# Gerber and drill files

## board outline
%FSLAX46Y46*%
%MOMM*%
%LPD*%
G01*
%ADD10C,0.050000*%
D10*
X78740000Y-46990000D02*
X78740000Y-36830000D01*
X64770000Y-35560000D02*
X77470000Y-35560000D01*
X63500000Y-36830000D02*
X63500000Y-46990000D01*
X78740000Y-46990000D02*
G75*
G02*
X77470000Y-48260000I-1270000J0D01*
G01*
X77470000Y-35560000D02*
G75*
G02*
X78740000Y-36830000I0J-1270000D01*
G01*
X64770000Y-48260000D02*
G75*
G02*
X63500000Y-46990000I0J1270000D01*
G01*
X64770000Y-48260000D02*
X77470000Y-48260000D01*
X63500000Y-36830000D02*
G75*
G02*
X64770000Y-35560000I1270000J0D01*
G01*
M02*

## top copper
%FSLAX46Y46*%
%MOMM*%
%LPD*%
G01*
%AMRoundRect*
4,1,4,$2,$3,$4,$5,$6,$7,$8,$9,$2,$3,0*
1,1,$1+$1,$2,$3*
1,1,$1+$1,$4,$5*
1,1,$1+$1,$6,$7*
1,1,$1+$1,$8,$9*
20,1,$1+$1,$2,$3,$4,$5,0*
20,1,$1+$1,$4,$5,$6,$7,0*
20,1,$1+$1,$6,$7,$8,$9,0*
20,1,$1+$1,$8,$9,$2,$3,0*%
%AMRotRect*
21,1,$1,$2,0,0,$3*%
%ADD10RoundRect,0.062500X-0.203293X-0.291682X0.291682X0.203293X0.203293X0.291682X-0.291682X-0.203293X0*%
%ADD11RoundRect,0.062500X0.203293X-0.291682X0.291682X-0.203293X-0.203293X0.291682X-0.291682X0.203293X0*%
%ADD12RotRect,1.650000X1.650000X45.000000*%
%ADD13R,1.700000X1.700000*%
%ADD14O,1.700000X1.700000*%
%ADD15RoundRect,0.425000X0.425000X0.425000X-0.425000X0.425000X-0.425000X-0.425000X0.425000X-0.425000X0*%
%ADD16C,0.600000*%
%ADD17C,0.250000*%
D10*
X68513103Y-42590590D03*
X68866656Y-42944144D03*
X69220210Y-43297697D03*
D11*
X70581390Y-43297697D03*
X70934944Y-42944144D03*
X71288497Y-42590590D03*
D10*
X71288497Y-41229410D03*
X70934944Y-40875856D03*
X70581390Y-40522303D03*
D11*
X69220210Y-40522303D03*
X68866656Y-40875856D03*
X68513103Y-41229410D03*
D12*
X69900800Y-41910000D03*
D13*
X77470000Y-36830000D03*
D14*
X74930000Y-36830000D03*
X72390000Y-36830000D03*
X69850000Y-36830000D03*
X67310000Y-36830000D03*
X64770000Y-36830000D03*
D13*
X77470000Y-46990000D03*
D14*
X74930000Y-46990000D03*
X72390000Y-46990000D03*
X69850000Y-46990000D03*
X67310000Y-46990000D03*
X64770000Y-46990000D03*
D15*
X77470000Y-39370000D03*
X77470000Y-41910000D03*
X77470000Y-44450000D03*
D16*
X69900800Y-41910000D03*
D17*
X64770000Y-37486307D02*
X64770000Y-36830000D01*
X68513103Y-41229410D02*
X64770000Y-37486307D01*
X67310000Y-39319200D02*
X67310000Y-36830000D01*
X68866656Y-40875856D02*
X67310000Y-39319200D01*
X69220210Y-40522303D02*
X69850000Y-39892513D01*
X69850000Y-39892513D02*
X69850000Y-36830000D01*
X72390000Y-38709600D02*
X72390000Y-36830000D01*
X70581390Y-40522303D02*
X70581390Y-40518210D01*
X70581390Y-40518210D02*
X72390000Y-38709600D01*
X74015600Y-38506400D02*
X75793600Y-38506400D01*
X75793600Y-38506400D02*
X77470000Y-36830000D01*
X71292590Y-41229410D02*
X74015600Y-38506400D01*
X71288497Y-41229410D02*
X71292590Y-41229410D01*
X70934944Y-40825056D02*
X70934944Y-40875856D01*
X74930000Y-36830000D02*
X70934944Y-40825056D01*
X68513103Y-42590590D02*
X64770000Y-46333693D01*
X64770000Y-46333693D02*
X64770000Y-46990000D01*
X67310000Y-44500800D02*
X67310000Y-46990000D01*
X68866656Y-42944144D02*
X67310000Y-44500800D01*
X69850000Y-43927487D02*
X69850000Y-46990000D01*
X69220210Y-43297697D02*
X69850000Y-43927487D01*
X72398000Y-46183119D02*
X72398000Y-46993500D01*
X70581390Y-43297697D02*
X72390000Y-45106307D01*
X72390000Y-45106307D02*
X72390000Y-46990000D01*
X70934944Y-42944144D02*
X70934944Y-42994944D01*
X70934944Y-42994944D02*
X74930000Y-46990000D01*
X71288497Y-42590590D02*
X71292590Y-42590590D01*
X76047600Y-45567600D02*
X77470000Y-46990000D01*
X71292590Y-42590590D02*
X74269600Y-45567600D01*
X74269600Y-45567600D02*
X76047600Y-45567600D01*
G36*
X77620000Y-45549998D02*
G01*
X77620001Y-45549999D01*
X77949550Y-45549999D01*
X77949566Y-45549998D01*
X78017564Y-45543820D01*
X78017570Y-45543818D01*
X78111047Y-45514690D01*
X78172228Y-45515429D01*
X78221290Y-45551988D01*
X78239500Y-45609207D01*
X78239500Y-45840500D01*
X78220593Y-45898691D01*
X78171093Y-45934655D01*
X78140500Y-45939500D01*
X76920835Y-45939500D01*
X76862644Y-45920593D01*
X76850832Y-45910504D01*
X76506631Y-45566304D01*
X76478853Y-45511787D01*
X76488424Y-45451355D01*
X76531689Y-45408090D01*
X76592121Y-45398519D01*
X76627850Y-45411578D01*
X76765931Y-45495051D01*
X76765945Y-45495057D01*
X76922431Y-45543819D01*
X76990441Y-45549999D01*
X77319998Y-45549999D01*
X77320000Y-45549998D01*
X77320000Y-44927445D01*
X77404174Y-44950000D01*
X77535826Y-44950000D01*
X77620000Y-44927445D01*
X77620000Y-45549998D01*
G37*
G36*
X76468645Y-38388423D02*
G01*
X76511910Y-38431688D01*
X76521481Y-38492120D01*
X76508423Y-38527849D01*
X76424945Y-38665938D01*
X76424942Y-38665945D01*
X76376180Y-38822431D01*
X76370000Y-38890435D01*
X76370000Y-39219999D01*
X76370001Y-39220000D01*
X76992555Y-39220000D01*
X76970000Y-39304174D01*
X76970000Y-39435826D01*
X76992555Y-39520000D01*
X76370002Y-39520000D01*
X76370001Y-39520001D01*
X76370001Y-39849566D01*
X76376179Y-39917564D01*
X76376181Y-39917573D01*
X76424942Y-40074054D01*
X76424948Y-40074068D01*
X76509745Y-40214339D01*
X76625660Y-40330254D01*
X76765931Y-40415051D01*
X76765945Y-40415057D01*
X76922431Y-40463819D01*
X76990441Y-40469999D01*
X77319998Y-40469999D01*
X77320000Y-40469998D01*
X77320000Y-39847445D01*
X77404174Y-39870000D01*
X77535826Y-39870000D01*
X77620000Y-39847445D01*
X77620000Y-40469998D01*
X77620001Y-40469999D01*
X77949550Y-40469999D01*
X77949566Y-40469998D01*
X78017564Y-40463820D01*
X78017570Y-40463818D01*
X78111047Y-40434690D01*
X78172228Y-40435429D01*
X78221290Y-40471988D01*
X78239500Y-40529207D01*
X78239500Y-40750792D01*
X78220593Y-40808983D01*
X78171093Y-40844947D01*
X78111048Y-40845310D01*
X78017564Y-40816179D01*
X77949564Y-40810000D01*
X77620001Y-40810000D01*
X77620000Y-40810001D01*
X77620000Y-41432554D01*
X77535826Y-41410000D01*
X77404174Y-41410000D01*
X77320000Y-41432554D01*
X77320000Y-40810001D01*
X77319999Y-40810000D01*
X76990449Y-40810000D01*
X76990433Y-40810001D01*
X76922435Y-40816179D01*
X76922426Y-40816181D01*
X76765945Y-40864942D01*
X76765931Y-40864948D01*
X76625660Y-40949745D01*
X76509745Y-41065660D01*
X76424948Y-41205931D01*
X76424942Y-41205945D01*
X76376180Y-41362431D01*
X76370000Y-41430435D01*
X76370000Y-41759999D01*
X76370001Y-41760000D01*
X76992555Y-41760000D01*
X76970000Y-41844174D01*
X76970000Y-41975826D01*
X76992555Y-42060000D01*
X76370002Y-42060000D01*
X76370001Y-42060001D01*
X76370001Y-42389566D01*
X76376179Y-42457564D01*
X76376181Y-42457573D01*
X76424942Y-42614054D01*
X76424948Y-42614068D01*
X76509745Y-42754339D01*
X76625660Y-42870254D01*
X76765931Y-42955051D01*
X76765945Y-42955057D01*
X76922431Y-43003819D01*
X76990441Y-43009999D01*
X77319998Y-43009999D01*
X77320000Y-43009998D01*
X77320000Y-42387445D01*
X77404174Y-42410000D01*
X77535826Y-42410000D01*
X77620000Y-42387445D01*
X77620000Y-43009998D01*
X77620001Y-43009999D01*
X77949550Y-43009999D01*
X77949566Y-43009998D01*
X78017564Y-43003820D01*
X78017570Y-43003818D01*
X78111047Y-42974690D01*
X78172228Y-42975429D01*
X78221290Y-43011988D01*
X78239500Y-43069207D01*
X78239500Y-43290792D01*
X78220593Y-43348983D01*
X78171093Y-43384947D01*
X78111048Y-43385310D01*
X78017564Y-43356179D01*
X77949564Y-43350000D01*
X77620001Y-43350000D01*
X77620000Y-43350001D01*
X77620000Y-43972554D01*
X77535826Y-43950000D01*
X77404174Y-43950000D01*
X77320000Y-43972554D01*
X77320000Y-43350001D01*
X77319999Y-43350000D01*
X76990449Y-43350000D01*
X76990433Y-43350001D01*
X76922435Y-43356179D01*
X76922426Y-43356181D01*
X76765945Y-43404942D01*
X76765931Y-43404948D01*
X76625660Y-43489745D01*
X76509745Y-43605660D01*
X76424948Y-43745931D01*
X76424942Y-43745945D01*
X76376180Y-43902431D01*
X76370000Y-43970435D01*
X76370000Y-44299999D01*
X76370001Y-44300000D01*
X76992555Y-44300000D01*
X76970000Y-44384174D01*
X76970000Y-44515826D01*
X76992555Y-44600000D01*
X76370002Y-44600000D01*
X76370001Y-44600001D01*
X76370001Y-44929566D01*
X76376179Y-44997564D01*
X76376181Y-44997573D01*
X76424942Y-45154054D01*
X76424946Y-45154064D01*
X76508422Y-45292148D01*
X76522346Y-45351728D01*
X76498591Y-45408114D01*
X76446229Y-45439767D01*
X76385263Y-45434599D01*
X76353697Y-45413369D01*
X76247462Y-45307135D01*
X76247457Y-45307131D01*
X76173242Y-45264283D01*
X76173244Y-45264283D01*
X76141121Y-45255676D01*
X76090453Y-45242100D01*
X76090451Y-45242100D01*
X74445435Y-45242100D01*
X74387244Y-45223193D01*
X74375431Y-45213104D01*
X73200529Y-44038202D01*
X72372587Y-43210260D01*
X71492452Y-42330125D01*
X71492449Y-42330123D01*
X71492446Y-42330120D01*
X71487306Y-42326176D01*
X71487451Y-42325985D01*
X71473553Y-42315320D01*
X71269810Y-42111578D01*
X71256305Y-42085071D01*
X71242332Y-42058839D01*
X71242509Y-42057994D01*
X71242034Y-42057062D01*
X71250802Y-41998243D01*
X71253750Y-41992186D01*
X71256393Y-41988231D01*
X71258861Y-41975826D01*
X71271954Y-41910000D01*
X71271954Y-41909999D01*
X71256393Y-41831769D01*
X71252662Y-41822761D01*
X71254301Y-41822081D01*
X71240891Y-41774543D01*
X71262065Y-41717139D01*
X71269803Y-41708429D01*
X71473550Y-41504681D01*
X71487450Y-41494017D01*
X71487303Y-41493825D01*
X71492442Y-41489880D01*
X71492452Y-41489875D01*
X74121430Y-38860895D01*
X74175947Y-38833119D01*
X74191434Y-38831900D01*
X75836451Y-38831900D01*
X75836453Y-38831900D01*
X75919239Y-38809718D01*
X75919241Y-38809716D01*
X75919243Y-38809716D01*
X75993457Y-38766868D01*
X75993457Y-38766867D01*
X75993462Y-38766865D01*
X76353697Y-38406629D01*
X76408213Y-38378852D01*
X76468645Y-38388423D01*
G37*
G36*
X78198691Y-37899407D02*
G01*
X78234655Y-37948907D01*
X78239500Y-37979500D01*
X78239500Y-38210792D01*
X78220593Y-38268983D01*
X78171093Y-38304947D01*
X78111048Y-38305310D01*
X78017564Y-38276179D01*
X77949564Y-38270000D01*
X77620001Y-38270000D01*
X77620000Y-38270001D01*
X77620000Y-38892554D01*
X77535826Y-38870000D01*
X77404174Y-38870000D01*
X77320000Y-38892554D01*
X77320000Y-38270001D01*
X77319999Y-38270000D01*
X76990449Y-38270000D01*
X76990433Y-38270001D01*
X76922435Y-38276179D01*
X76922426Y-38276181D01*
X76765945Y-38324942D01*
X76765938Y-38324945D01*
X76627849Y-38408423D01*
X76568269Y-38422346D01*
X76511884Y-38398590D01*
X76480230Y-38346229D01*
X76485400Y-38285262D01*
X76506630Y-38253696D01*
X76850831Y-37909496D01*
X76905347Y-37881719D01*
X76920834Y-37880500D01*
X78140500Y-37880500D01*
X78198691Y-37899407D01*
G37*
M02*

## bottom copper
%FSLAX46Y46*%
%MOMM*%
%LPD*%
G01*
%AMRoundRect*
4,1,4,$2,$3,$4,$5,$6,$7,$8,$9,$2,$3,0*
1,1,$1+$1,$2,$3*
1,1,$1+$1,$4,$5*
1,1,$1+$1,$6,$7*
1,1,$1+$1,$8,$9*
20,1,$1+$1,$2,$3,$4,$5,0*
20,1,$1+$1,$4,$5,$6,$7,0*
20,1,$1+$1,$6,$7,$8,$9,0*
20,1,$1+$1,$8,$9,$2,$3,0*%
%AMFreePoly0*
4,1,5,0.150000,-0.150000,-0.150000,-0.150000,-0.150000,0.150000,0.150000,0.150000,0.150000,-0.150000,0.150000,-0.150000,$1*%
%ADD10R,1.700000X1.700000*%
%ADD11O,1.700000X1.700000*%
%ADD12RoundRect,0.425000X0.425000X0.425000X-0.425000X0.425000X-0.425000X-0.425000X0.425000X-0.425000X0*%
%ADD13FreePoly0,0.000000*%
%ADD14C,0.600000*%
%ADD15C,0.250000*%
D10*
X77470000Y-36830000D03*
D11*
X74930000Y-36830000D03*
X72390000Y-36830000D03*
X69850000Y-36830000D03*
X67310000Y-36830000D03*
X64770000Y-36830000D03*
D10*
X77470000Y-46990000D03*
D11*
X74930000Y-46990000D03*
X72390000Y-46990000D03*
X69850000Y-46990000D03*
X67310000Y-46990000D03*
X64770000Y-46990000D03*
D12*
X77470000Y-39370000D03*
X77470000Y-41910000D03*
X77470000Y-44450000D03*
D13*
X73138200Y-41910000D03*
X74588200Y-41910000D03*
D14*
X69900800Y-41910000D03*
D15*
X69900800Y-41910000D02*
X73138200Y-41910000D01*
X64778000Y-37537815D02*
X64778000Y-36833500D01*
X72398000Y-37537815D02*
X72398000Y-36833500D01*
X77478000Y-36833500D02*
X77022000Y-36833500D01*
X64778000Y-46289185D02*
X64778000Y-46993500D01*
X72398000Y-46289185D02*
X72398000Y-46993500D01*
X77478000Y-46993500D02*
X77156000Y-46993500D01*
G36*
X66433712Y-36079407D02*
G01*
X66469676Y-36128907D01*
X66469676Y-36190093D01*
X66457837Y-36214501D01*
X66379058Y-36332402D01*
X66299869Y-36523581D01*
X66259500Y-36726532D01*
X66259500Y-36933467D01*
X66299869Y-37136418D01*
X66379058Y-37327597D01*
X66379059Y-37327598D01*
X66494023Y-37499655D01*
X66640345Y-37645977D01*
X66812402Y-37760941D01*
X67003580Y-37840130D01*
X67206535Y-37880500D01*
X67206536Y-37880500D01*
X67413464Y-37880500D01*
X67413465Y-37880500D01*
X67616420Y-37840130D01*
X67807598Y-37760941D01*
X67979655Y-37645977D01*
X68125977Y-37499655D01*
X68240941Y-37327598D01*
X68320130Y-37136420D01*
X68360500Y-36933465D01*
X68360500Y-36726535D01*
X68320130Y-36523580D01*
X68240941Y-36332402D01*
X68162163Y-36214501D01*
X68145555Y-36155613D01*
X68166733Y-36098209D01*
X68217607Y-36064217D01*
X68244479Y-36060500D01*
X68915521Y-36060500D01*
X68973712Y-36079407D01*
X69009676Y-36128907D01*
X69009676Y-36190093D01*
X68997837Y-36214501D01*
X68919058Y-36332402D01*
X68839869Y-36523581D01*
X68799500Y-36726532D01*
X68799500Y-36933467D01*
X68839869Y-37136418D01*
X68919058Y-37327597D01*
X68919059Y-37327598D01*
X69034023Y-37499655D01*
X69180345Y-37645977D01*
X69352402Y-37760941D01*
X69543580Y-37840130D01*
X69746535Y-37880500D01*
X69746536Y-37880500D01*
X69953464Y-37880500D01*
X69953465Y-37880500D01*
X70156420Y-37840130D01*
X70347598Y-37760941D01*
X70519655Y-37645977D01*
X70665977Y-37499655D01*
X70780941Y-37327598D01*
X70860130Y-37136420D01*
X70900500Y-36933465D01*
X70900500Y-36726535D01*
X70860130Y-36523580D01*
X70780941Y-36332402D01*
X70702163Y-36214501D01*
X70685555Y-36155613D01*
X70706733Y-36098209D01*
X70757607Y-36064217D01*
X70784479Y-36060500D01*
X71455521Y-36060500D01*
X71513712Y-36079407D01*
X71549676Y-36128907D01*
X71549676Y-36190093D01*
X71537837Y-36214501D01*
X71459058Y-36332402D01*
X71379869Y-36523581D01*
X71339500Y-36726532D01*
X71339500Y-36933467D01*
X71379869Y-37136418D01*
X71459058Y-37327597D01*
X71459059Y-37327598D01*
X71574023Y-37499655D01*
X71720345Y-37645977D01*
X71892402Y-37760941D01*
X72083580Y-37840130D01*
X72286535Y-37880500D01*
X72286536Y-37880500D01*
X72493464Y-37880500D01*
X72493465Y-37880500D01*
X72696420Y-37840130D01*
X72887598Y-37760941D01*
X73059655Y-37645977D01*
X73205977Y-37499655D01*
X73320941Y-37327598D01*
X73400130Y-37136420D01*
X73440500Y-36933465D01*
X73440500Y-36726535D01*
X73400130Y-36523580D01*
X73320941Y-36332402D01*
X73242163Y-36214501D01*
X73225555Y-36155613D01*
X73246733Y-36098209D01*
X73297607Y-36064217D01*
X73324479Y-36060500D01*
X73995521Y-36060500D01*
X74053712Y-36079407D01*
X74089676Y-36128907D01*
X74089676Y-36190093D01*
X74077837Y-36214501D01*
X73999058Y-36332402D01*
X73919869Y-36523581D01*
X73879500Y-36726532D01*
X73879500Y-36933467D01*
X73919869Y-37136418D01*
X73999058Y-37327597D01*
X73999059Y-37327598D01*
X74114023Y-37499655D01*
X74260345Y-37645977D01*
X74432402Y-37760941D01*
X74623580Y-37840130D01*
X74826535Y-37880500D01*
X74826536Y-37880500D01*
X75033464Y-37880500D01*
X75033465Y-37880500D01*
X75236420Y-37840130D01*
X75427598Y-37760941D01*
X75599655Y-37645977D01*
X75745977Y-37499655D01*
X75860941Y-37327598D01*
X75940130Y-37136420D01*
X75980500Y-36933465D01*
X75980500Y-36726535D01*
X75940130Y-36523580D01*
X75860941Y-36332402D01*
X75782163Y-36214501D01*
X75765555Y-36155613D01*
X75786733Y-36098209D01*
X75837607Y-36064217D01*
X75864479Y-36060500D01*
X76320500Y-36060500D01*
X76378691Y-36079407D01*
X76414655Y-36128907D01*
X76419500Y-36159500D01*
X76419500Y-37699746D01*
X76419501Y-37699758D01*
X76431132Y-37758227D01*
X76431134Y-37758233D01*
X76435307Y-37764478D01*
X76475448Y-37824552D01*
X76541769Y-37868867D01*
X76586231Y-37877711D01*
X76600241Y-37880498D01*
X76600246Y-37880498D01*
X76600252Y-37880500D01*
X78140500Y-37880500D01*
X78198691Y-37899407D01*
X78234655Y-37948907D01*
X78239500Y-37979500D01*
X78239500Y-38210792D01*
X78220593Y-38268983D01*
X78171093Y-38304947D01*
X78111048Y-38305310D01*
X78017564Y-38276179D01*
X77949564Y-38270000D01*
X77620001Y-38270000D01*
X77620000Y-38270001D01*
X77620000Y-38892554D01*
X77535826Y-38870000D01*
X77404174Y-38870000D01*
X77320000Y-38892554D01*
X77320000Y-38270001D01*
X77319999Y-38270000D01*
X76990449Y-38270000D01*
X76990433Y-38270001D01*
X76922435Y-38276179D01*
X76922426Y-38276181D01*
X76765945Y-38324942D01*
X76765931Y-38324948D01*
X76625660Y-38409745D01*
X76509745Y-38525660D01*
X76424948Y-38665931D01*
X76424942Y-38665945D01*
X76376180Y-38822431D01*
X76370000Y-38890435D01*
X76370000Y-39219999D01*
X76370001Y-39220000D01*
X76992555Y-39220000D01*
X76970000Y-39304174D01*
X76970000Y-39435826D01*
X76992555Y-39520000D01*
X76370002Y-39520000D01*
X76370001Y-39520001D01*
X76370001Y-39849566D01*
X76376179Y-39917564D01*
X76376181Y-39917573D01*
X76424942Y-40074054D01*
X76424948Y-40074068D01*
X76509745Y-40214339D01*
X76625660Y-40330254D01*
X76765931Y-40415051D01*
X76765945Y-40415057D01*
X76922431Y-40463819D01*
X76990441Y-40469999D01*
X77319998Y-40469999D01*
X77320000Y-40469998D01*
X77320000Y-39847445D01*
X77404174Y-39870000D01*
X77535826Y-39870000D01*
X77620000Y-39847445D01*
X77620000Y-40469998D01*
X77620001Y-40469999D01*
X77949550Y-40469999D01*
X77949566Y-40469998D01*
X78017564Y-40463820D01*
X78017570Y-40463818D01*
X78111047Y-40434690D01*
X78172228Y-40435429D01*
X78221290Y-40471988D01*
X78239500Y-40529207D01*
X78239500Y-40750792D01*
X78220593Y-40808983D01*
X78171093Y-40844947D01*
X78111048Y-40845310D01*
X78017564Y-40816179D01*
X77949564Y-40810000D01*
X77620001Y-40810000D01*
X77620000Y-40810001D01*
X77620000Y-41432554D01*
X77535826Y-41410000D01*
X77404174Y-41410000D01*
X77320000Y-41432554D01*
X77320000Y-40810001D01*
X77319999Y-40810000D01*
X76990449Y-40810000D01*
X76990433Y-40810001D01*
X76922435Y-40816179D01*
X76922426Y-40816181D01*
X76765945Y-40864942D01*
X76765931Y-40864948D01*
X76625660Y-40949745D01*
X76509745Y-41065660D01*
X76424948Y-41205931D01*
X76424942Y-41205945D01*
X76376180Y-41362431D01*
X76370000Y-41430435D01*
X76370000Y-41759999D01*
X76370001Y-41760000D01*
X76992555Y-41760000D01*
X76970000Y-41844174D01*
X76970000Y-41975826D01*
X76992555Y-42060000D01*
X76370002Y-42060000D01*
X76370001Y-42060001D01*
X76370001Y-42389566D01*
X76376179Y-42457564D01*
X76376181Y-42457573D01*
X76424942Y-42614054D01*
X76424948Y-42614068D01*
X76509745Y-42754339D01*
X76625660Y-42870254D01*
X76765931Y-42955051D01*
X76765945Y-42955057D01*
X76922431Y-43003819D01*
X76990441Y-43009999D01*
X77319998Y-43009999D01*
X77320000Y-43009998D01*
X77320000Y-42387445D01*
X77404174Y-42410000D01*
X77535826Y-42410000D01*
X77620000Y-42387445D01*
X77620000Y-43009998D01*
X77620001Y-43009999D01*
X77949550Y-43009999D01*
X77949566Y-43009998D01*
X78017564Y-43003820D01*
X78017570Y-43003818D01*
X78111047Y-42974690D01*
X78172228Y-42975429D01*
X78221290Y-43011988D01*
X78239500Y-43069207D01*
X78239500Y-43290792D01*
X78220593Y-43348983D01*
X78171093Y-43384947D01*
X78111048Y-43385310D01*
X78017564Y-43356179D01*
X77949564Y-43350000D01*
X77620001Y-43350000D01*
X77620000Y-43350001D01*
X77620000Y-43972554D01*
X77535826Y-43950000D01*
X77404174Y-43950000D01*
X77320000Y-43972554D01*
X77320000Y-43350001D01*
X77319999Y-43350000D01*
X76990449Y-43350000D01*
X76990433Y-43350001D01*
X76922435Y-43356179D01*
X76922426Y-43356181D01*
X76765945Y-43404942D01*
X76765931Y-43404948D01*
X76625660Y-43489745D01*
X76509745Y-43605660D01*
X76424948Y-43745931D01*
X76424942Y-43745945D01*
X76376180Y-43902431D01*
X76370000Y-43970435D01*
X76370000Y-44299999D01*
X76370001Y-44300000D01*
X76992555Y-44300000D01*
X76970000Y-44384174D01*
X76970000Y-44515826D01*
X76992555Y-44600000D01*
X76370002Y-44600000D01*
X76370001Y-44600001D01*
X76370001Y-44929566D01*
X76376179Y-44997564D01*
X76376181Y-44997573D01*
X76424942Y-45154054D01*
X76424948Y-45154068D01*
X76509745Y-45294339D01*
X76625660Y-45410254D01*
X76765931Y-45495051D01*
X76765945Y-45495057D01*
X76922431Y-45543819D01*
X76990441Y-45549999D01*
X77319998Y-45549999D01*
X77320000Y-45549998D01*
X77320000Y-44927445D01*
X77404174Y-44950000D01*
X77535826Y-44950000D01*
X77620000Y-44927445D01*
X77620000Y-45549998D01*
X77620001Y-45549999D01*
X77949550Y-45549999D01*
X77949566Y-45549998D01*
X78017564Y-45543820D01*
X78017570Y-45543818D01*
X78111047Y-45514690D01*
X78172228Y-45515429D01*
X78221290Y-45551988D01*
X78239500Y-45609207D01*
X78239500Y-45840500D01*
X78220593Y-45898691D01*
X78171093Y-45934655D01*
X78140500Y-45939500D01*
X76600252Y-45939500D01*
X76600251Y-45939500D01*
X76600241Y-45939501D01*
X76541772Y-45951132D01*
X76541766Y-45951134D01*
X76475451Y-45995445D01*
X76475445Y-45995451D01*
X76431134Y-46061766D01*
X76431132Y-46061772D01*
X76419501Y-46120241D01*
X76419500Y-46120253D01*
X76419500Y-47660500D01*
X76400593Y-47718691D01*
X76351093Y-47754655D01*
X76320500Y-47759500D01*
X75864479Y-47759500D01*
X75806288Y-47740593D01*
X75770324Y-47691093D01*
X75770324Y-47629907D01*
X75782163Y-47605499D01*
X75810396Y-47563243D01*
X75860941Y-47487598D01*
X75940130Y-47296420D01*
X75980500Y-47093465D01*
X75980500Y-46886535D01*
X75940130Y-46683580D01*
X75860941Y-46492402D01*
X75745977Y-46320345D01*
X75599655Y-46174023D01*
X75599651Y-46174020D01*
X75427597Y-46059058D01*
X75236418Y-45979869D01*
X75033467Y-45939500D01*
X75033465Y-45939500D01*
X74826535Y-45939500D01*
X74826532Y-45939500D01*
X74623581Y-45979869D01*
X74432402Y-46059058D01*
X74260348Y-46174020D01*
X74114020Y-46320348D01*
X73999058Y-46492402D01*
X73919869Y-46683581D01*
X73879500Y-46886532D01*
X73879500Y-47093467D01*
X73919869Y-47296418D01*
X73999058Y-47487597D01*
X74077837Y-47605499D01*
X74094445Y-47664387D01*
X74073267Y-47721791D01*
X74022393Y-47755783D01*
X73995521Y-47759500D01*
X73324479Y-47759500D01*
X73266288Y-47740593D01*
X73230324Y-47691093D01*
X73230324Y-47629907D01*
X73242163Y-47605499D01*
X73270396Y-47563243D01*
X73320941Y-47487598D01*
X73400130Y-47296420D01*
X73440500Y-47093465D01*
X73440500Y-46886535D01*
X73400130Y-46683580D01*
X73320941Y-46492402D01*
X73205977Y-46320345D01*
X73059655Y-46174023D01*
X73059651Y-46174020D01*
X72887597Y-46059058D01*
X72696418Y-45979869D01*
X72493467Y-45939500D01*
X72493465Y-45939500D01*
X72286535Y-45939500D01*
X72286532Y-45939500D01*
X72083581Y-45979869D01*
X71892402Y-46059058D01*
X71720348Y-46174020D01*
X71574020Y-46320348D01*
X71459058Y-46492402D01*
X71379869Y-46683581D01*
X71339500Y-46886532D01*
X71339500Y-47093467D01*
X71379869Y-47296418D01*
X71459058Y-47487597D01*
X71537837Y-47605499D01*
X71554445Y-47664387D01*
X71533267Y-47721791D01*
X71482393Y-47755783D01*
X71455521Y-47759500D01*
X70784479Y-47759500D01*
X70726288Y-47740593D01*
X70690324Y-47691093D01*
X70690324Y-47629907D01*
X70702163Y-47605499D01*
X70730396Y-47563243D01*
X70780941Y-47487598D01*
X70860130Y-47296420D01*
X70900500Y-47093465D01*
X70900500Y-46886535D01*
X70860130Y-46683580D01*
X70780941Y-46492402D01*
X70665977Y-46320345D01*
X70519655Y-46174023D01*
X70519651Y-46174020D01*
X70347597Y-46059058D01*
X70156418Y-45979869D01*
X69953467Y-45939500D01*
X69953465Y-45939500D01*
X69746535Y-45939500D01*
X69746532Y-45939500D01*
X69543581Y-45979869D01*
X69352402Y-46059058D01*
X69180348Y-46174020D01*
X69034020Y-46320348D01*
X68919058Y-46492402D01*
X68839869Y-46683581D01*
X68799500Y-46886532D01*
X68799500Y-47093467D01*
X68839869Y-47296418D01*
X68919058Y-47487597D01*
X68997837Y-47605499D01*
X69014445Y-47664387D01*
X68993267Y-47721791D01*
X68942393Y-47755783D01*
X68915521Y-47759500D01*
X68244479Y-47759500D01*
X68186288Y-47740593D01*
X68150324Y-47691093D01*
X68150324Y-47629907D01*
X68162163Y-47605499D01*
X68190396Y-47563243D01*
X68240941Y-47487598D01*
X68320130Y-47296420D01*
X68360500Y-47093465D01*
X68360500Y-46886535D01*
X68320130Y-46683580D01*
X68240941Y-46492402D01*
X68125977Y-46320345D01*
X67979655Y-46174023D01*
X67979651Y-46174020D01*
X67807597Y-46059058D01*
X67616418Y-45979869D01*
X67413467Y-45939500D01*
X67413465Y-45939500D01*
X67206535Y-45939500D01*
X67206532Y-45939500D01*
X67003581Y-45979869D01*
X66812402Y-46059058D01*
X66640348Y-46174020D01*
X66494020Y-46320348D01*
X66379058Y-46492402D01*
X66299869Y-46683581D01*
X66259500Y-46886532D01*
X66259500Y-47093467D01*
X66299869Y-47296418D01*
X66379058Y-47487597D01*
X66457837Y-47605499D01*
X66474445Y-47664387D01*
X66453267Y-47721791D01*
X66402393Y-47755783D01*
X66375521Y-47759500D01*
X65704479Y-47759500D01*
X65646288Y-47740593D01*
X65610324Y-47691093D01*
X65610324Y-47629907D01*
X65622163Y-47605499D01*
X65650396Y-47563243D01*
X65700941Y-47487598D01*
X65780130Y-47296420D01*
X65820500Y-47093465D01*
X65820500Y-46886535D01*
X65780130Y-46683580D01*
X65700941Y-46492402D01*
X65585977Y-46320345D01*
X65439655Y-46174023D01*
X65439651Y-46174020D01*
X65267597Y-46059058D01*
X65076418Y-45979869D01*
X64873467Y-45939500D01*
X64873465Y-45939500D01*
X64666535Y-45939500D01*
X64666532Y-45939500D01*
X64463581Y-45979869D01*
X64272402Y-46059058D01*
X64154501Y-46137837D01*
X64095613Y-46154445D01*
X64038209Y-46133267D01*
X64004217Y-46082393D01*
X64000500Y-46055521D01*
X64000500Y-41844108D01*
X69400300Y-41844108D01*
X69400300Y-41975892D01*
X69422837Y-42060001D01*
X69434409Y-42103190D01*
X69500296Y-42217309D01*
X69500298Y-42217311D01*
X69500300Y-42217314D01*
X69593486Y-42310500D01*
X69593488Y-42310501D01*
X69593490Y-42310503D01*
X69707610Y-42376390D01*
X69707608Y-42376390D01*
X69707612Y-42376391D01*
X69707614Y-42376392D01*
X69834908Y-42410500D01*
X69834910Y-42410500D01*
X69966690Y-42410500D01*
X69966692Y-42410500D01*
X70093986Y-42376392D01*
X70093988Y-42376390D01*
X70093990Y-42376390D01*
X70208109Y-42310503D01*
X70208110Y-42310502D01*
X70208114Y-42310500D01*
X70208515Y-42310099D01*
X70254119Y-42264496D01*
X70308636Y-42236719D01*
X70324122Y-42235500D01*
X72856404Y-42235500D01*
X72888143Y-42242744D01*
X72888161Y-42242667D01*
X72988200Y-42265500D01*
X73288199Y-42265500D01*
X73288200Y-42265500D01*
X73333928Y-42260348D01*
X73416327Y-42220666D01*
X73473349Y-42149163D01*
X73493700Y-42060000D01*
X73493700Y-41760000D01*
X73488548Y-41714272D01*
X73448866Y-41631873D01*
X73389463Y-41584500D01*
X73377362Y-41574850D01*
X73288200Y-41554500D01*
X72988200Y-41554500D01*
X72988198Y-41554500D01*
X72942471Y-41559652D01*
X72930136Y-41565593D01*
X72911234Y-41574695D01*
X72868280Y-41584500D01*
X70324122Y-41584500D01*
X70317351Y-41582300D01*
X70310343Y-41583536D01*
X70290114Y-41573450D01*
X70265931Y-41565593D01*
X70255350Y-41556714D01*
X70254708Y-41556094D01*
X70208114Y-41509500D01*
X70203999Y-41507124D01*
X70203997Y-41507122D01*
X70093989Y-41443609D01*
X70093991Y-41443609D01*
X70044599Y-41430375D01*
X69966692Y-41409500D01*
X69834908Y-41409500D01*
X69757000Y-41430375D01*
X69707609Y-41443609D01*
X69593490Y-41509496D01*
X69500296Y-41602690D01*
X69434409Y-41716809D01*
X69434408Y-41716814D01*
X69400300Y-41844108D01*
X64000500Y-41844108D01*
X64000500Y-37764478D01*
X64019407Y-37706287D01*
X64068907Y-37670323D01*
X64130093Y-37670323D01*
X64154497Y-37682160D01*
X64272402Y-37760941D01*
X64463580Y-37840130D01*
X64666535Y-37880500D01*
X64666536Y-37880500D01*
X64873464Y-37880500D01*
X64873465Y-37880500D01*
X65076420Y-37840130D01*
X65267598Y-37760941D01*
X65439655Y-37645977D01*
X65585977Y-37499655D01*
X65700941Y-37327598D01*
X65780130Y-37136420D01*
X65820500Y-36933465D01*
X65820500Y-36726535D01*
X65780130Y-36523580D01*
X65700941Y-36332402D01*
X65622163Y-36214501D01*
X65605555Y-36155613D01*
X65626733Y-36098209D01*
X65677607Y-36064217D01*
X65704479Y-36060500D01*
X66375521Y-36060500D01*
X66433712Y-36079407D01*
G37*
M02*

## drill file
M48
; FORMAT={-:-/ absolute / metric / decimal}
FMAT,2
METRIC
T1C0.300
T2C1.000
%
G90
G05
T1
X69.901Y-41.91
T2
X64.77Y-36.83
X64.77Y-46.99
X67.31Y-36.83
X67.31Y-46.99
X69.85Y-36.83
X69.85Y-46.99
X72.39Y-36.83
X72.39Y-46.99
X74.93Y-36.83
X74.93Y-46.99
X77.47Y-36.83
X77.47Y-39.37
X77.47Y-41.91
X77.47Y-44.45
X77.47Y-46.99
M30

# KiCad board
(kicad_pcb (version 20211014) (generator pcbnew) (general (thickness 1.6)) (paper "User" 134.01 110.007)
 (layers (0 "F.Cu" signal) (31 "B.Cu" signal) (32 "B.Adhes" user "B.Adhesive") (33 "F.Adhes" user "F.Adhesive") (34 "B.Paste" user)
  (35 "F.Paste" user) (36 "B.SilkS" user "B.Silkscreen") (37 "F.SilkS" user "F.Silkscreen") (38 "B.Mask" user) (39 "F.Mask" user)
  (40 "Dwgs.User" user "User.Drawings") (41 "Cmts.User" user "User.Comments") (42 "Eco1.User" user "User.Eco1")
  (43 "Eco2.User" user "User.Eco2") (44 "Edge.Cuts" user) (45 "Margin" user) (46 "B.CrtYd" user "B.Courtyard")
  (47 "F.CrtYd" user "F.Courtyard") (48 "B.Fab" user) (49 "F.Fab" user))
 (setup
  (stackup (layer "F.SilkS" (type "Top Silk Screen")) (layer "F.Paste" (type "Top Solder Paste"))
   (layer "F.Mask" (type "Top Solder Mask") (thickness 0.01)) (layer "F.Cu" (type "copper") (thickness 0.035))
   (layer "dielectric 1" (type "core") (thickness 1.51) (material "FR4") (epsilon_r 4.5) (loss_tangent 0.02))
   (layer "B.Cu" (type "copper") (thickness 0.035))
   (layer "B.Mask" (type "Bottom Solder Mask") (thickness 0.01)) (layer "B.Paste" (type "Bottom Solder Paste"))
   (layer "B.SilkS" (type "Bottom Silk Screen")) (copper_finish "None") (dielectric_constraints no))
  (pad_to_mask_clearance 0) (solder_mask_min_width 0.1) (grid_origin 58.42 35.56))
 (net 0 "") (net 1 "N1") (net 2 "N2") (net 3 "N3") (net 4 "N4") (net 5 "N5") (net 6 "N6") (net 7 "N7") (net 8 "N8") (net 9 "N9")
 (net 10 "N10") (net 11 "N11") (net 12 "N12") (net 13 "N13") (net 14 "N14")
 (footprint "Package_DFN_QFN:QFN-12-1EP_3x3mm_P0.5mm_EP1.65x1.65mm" (layer "F.Cu") (at 69.9008 41.91 45)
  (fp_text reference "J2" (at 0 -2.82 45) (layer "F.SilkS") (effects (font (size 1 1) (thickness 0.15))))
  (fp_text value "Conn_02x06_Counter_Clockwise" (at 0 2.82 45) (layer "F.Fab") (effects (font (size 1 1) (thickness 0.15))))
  (pad "" smd roundrect (at -0.41 -0.41 45) (size 0.67 0.67) (layers "F.Paste") (roundrect_rratio 0.25))
  (pad "" smd roundrect (at 0.41 -0.41 45) (size 0.67 0.67) (layers "F.Paste") (roundrect_rratio 0.25))
  (pad "" smd roundrect (at 0.41 0.41 45) (size 0.67 0.67) (layers "F.Paste") (roundrect_rratio 0.25))
  (pad "" smd roundrect (at -0.41 0.41 45) (size 0.67 0.67) (layers "F.Paste") (roundrect_rratio 0.25))
  (pad "1" smd roundrect (at -1.4625 -0.5 45) (size 0.825 0.25) (layers "F.Cu" "F.Paste" "F.Mask") (roundrect_rratio 0.25) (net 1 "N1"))
  (pad "2" smd roundrect (at -1.4625 0 45) (size 0.825 0.25) (layers "F.Cu" "F.Paste" "F.Mask") (roundrect_rratio 0.25) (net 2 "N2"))
  (pad "3" smd roundrect (at -1.4625 0.5 45) (size 0.825 0.25) (layers "F.Cu" "F.Paste" "F.Mask") (roundrect_rratio 0.25) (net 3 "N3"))
  (pad "4" smd roundrect (at -0.5 1.4625 45) (size 0.25 0.825) (layers "F.Cu" "F.Paste" "F.Mask") (roundrect_rratio 0.25) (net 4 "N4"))
  (pad "5" smd roundrect (at 0 1.4625 45) (size 0.25 0.825) (layers "F.Cu" "F.Paste" "F.Mask") (roundrect_rratio 0.25) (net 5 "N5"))
  (pad "6" smd roundrect (at 0.5 1.4625 45) (size 0.25 0.825) (layers "F.Cu" "F.Paste" "F.Mask") (roundrect_rratio 0.25) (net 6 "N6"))
  (pad "7" smd roundrect (at 1.4625 0.5 45) (size 0.825 0.25) (layers "F.Cu" "F.Paste" "F.Mask") (roundrect_rratio 0.25) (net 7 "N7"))
  (pad "8" smd roundrect (at 1.4625 0 45) (size 0.825 0.25) (layers "F.Cu" "F.Paste" "F.Mask") (roundrect_rratio 0.25) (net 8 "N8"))
  (pad "9" smd roundrect (at 1.4625 -0.5 45) (size 0.825 0.25) (layers "F.Cu" "F.Paste" "F.Mask") (roundrect_rratio 0.25) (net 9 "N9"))
  (pad "10" smd roundrect (at 0.5 -1.4625 45) (size 0.25 0.825) (layers "F.Cu" "F.Paste" "F.Mask") (roundrect_rratio 0.25) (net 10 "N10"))
  (pad "11" smd roundrect (at 0 -1.4625 45) (size 0.25 0.825) (layers "F.Cu" "F.Paste" "F.Mask") (roundrect_rratio 0.25) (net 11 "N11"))
  (pad "12" smd roundrect (at -0.5 -1.4625 45) (size 0.25 0.825) (layers "F.Cu" "F.Paste" "F.Mask") (roundrect_rratio 0.25) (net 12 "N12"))
  (pad "13" smd rect (at 0 0 45) (size 1.65 1.65) (layers "F.Cu" "F.Mask") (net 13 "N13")))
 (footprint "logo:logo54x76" (layer "F.Cu") (at 65.532 41.9608)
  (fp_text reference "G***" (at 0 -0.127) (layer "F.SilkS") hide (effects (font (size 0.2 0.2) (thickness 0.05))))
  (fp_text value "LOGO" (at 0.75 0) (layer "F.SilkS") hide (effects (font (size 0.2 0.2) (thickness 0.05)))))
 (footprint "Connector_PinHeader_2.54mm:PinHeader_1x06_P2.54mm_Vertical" (layer "B.Cu") (at 77.47 36.83 90)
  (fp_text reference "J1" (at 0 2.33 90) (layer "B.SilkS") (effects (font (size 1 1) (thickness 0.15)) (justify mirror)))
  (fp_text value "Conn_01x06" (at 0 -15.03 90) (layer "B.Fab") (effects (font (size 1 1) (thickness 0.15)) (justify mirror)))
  (pad "1" thru_hole rect (at 0 0 90) (size 1.7 1.7) (drill 1) (layers *.Cu *.Mask) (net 7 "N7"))
  (pad "2" thru_hole oval (at 0 -2.54 90) (size 1.7 1.7) (drill 1) (layers *.Cu *.Mask) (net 8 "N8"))
  (pad "3" thru_hole oval (at 0 -5.08 90) (size 1.7 1.7) (drill 1) (layers *.Cu *.Mask) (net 9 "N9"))
  (pad "4" thru_hole oval (at 0 -7.62 90) (size 1.7 1.7) (drill 1) (layers *.Cu *.Mask) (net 10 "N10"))
  (pad "5" thru_hole oval (at 0 -10.16 90) (size 1.7 1.7) (drill 1) (layers *.Cu *.Mask) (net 11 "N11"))
  (pad "6" thru_hole oval (at 0 -12.7 90) (size 1.7 1.7) (drill 1) (layers *.Cu *.Mask) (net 12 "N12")))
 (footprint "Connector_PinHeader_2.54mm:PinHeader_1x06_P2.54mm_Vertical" (layer "B.Cu") (at 77.47 46.99 90)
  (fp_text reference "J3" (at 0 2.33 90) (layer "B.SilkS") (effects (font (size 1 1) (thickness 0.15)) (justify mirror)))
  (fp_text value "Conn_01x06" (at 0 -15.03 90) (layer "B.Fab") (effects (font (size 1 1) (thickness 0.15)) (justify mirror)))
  (pad "1" thru_hole rect (at 0 0 90) (size 1.7 1.7) (drill 1) (layers *.Cu *.Mask) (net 6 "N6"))
  (pad "2" thru_hole oval (at 0 -2.54 90) (size 1.7 1.7) (drill 1) (layers *.Cu *.Mask) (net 5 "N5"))
  (pad "3" thru_hole oval (at 0 -5.08 90) (size 1.7 1.7) (drill 1) (layers *.Cu *.Mask) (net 4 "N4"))
  (pad "4" thru_hole oval (at 0 -7.62 90) (size 1.7 1.7) (drill 1) (layers *.Cu *.Mask) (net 3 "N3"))
  (pad "5" thru_hole oval (at 0 -10.16 90) (size 1.7 1.7) (drill 1) (layers *.Cu *.Mask) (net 2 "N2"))
  (pad "6" thru_hole oval (at 0 -12.7 90) (size 1.7 1.7) (drill 1) (layers *.Cu *.Mask) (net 1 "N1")))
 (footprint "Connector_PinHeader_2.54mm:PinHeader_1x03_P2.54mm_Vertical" (layer "B.Cu") (at 77.47 39.37 180)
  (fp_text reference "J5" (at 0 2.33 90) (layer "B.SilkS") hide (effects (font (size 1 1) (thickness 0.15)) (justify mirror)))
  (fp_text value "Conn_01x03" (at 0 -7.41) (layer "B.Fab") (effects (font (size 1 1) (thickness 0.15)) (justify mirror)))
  (pad "1" thru_hole roundrect locked (at 0 0 180) (size 1.7 1.7) (drill 1) (layers *.Cu *.Mask) (roundrect_rratio 0.25) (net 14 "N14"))
  (pad "2" thru_hole roundrect locked (at 0 -2.54 180) (size 1.7 1.7) (drill 1) (layers *.Cu *.Mask) (roundrect_rratio 0.25) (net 14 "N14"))
  (pad "3" thru_hole roundrect locked (at 0 -5.08 180) (size 1.7 1.7) (drill 1) (layers *.Cu *.Mask) (roundrect_rratio 0.25) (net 14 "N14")))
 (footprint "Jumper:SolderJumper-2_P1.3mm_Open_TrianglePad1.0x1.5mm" (layer "B.Cu") (at 73.8632 41.91)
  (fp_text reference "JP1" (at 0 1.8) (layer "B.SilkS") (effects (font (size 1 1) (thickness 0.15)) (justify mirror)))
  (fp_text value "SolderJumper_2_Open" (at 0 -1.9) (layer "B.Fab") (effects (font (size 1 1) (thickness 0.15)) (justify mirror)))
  (pad "1" smd custom (at -0.725 0) (size 0.3 0.3) (layers "B.Cu" "B.Mask") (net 13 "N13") (zone_connect 2)
   (options (clearance outline) (anchor rect)) (primitives))
  (pad "2" smd custom (at 0.725 0) (size 0.3 0.3) (layers "B.Cu" "B.Mask") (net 14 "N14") (zone_connect 2)
   (options (clearance outline) (anchor rect)) (primitives)))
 (gr_line (start 78.74 46.99) (end 78.74 36.83) (layer "Edge.Cuts") (width 0.05))
 (gr_line (start 64.77 35.56) (end 77.47 35.56) (layer "Edge.Cuts") (width 0.05))
 (gr_line (start 63.5 36.83) (end 63.5 46.99) (layer "Edge.Cuts") (width 0.05))
 (gr_arc (start 78.74 46.99) (mid 78.368026 47.888026) (end 77.47 48.26) (layer "Edge.Cuts") (width 0.05))
 (gr_arc (start 77.47 35.56) (mid 78.368026 35.931974) (end 78.74 36.83) (layer "Edge.Cuts") (width 0.05))
 (gr_arc (start 64.77 48.26) (mid 63.871974 47.888026) (end 63.5 46.99) (layer "Edge.Cuts") (width 0.05))
 (gr_line (start 64.77 48.26) (end 77.47 48.26) (layer "Edge.Cuts") (width 0.05))
 (gr_arc (start 63.5 36.83) (mid 63.871974 35.931974) (end 64.77 35.56) (layer "Edge.Cuts") (width 0.05))
 (via (at 69.9008 41.91) (size 0.6) (drill 0.3) (layers "F.Cu" "B.Cu") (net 13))
 (segment (start 69.9008 41.91) (end 73.1382 41.91) (width 0.25) (layer "B.Cu") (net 13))
 (segment (start 64.77 37.486307) (end 64.77 36.83) (width 0.25) (layer "F.Cu") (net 12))
 (segment (start 68.513103 41.22941) (end 64.77 37.486307) (width 0.25) (layer "F.Cu") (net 12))
 (segment (start 64.778 37.537815) (end 64.778 36.8335) (width 0.25) (layer "B.Cu") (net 12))
 (segment (start 67.31 39.3192) (end 67.31 36.83) (width 0.25) (layer "F.Cu") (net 11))
 (segment (start 68.866656 40.875856) (end 67.31 39.3192) (width 0.25) (layer "F.Cu") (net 11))
 (segment (start 69.22021 40.522303) (end 69.85 39.892513) (width 0.25) (layer "F.Cu") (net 10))
 (segment (start 69.85 39.892513) (end 69.85 36.83) (width 0.25) (layer "F.Cu") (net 10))
 (segment (start 72.39 38.7096) (end 72.39 36.83) (width 0.25) (layer "F.Cu") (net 9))
 (segment (start 70.58139 40.522303) (end 70.58139 40.51821) (width 0.25) (layer "F.Cu") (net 9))
 (segment (start 70.58139 40.51821) (end 72.39 38.7096) (width 0.25) (layer "F.Cu") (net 9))
 (segment (start 72.398 37.537815) (end 72.398 36.8335) (width 0.25) (layer "B.Cu") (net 9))
 (segment (start 74.0156 38.5064) (end 75.7936 38.5064) (width 0.25) (layer "F.Cu") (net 7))
 (segment (start 75.7936 38.5064) (end 77.47 36.83) (width 0.25) (layer "F.Cu") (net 7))
 (segment (start 71.29259 41.22941) (end 74.0156 38.5064) (width 0.25) (layer "F.Cu") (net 7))
 (segment (start 71.288497 41.22941) (end 71.29259 41.22941) (width 0.25) (layer "F.Cu") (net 7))
 (segment (start 77.478 36.8335) (end 77.022 36.8335) (width 0.25) (layer "B.Cu") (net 7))
 (segment (start 70.934944 40.825056) (end 70.934944 40.875856) (width 0.25) (layer "F.Cu") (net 8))
 (segment (start 74.93 36.83) (end 70.934944 40.825056) (width 0.25) (layer "F.Cu") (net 8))
 (segment (start 68.513103 42.59059) (end 64.77 46.333693) (width 0.25) (layer "F.Cu") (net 1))
 (segment (start 64.77 46.333693) (end 64.77 46.99) (width 0.25) (layer "F.Cu") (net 1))
 (segment (start 64.778 46.289185) (end 64.778 46.9935) (width 0.25) (layer "B.Cu") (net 1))
 (segment (start 67.31 44.5008) (end 67.31 46.99) (width 0.25) (layer "F.Cu") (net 2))
 (segment (start 68.866656 42.944144) (end 67.31 44.5008) (width 0.25) (layer "F.Cu") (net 2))
 (segment (start 69.85 43.927487) (end 69.85 46.99) (width 0.25) (layer "F.Cu") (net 3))
 (segment (start 69.22021 43.297697) (end 69.85 43.927487) (width 0.25) (layer "F.Cu") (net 3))
 (segment (start 72.398 46.183119) (end 72.398 46.9935) (width 0.25) (layer "F.Cu") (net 4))
 (segment (start 70.58139 43.297697) (end 72.39 45.106307) (width 0.25) (layer "F.Cu") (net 4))
 (segment (start 72.39 45.106307) (end 72.39 46.99) (width 0.25) (layer "F.Cu") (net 4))
 (segment (start 72.398 46.289185) (end 72.398 46.9935) (width 0.25) (layer "B.Cu") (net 4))
 (segment (start 70.934944 42.944144) (end 70.934944 42.994944) (width 0.25) (layer "F.Cu") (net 5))
 (segment (start 70.934944 42.994944) (end 74.93 46.99) (width 0.25) (layer "F.Cu") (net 5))
 (segment (start 71.288497 42.59059) (end 71.29259 42.59059) (width 0.25) (layer "F.Cu") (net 6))
 (segment (start 76.0476 45.5676) (end 77.47 46.99) (width 0.25) (layer "F.Cu") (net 6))
 (segment (start 71.29259 42.59059) (end 74.2696 45.5676) (width 0.25) (layer "F.Cu") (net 6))
 (segment (start 74.2696 45.5676) (end 76.0476 45.5676) (width 0.25) (layer "F.Cu") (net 6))
 (segment (start 77.478 46.9935) (end 77.156 46.9935) (width 0.25) (layer "B.Cu") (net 6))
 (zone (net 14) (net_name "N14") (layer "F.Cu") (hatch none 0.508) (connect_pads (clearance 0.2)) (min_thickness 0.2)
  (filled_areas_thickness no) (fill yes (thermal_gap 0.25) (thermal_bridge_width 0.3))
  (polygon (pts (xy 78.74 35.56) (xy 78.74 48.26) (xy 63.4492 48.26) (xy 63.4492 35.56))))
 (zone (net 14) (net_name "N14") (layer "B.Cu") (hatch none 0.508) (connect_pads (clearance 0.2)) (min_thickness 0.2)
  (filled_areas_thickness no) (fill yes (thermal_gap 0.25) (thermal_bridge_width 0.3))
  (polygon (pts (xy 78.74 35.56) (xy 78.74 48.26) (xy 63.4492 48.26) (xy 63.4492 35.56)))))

